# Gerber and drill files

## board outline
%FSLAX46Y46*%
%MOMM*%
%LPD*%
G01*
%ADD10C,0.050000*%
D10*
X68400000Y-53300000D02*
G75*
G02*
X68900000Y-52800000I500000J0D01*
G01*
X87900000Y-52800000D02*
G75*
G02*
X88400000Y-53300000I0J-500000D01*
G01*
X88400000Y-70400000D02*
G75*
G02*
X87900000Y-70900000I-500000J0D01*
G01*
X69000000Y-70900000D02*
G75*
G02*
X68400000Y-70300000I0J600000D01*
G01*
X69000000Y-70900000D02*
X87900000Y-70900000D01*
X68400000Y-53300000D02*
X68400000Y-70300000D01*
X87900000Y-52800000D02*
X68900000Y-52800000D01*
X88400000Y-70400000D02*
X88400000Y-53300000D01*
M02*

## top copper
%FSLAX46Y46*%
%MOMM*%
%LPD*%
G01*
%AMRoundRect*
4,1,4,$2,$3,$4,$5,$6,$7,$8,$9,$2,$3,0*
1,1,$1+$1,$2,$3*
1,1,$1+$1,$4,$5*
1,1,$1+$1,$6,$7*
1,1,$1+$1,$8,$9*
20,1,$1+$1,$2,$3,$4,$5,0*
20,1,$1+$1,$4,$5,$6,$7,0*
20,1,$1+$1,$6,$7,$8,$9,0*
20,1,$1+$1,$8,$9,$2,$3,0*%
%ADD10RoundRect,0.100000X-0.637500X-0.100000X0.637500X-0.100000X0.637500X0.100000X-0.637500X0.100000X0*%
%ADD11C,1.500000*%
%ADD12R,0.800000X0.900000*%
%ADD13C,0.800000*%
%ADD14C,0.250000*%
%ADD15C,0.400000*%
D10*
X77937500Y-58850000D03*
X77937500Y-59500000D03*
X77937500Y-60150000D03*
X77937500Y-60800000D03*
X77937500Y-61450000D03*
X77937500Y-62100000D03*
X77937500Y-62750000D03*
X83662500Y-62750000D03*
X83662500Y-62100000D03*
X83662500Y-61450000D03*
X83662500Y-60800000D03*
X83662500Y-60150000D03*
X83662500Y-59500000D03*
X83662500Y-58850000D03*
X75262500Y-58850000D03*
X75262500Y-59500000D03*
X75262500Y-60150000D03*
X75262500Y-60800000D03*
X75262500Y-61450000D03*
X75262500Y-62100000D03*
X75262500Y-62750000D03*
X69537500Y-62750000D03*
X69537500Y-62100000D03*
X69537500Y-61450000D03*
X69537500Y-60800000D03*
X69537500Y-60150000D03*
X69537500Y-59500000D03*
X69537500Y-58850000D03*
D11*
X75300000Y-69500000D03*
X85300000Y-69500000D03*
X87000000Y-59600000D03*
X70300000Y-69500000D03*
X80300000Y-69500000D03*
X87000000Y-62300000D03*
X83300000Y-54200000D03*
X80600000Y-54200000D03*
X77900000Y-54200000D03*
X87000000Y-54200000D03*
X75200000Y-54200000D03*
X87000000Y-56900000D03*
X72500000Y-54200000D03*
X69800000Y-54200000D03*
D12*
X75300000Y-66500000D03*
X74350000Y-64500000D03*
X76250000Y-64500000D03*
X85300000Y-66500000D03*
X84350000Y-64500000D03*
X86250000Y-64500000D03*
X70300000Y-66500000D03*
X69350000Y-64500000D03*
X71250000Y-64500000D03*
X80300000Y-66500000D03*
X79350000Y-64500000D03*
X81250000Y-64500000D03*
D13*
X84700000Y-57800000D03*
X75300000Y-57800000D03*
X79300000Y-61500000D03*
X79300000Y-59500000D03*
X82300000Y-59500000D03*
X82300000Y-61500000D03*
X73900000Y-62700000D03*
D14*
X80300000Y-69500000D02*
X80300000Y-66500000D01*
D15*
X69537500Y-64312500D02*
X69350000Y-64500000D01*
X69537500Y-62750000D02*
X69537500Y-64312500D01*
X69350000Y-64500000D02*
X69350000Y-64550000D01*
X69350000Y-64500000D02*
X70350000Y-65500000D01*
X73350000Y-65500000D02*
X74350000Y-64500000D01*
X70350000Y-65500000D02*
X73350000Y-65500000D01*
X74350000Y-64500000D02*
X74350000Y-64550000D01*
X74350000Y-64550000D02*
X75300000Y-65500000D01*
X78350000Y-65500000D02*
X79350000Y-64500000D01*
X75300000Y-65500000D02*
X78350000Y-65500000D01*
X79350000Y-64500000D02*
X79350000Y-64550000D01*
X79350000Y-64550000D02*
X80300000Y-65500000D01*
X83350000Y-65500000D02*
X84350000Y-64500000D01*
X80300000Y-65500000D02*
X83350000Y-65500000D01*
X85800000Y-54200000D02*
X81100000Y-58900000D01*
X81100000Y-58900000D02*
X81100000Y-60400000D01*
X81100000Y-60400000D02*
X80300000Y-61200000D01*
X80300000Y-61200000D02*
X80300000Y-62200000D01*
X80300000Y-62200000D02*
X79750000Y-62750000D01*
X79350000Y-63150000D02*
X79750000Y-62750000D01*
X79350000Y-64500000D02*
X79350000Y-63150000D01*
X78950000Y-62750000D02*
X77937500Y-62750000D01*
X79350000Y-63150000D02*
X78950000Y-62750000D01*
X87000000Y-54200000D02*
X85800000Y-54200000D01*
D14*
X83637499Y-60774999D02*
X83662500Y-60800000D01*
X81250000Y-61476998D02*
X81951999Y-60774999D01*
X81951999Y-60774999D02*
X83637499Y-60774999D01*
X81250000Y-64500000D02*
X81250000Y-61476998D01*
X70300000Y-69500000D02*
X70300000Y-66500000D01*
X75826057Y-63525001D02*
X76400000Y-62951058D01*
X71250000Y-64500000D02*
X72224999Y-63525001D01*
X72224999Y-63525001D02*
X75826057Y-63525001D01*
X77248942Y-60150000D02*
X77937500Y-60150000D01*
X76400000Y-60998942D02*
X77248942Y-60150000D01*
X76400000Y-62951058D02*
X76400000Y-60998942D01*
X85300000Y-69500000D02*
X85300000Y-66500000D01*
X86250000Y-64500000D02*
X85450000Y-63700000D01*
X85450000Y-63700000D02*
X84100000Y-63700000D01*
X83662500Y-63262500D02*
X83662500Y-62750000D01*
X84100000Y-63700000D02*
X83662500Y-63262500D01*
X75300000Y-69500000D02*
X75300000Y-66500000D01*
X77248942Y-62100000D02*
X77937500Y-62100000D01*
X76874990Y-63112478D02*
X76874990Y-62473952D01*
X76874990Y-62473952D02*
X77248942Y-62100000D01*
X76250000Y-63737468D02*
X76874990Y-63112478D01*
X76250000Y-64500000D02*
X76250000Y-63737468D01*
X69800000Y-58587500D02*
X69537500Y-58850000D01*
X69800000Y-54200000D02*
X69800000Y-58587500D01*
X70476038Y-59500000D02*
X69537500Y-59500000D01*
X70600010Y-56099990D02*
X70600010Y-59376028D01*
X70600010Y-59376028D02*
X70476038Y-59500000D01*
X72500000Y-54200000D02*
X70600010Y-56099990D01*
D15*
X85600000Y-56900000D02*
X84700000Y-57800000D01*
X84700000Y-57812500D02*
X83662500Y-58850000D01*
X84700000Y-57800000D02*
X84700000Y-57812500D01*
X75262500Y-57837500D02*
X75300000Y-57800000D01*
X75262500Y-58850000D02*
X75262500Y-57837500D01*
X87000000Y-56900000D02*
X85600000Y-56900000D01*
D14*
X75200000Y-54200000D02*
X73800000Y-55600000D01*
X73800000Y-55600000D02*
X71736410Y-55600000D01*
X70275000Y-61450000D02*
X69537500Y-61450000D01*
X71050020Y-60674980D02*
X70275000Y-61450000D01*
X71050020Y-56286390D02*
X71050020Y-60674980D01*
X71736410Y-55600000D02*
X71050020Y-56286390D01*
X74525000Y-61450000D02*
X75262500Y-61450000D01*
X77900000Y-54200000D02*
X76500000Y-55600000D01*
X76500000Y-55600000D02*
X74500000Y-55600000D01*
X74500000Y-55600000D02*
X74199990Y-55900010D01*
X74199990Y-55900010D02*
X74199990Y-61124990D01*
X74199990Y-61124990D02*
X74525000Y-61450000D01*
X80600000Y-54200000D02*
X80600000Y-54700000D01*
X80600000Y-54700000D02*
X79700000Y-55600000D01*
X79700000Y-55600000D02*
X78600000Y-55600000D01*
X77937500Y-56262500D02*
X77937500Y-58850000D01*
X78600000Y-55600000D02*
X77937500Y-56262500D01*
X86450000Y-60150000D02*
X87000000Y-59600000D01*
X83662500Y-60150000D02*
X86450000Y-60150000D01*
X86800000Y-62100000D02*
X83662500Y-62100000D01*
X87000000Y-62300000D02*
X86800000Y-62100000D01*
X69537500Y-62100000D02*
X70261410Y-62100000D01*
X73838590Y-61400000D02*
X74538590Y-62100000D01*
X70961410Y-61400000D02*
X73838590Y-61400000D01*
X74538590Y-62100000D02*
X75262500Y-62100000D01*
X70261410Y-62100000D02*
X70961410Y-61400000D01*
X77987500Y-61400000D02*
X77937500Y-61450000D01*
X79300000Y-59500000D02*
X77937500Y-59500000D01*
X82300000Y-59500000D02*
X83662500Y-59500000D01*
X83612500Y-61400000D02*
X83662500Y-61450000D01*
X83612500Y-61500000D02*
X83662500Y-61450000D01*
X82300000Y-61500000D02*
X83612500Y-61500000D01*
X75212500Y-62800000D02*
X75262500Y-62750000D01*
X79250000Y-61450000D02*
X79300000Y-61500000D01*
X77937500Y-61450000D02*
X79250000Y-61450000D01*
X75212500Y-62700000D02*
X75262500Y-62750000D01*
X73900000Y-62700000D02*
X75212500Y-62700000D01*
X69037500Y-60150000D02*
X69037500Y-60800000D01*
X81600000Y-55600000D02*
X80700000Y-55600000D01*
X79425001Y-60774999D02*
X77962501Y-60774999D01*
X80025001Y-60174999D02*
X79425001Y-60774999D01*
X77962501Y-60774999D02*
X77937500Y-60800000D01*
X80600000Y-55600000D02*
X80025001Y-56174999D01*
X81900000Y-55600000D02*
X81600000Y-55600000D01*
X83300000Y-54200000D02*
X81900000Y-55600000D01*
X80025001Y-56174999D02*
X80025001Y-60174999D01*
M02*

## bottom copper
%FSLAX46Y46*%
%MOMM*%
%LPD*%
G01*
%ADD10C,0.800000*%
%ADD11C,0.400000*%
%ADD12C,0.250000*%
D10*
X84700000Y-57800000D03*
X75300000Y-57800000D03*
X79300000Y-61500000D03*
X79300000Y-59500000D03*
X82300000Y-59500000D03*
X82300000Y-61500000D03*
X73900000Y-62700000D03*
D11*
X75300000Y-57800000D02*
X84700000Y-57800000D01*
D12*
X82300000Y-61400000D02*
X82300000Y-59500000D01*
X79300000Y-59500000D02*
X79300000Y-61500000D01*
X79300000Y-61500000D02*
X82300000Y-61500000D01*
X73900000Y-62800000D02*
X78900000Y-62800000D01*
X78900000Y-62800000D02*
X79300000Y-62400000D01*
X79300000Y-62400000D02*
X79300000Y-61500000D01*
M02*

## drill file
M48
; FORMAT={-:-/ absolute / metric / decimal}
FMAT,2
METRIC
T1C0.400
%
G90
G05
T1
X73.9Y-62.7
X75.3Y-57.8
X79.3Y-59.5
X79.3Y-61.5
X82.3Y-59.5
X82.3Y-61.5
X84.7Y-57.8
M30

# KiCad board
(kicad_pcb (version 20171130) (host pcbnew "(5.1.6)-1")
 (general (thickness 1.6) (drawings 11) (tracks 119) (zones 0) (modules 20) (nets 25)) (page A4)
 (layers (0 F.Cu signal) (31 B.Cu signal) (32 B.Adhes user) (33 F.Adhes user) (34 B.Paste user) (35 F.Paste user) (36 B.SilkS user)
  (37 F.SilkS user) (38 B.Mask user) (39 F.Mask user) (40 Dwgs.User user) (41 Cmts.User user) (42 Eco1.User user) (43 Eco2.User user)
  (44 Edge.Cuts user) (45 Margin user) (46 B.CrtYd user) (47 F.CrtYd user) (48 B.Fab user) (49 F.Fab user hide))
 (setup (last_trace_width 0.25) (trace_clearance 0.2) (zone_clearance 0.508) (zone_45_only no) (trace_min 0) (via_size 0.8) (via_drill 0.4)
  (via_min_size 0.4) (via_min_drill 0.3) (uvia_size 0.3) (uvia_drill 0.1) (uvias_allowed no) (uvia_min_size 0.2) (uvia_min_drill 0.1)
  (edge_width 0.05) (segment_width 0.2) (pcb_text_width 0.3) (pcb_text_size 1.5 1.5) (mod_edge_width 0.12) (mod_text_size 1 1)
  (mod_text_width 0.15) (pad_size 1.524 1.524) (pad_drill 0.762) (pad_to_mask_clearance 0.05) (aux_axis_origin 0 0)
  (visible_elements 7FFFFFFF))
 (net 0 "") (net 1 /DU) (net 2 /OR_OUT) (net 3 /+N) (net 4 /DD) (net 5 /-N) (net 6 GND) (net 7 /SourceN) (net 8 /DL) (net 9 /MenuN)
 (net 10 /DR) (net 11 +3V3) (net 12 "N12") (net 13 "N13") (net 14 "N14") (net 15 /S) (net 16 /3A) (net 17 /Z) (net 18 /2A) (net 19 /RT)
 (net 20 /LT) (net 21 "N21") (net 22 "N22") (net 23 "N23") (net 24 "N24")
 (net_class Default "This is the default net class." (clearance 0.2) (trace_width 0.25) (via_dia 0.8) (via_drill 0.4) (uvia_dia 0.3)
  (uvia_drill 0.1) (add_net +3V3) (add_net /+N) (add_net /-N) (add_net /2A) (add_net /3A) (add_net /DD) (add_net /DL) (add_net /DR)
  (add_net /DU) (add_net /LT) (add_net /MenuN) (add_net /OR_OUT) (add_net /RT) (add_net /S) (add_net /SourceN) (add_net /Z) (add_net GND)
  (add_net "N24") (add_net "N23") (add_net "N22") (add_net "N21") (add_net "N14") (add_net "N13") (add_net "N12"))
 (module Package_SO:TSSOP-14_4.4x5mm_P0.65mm (layer F.Cu) (at 80.8 60.8)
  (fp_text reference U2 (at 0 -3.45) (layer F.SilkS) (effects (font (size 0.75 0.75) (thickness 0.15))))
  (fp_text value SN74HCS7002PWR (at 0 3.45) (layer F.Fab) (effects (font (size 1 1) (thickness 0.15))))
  (pad 1 smd roundrect (at -2.8625 -1.95) (size 1.475 0.4) (layers F.Cu F.Paste F.Mask) (roundrect_rratio 0.25) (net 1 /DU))
  (pad 2 smd roundrect (at -2.8625 -1.3) (size 1.475 0.4) (layers F.Cu F.Paste F.Mask) (roundrect_rratio 0.25) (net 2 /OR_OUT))
  (pad 3 smd roundrect (at -2.8625 -0.65) (size 1.475 0.4) (layers F.Cu F.Paste F.Mask) (roundrect_rratio 0.25) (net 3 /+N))
  (pad 4 smd roundrect (at -2.8625 0) (size 1.475 0.4) (layers F.Cu F.Paste F.Mask) (roundrect_rratio 0.25) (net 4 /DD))
  (pad 5 smd roundrect (at -2.8625 0.65) (size 1.475 0.4) (layers F.Cu F.Paste F.Mask) (roundrect_rratio 0.25) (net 2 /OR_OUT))
  (pad 6 smd roundrect (at -2.8625 1.3) (size 1.475 0.4) (layers F.Cu F.Paste F.Mask) (roundrect_rratio 0.25) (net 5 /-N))
  (pad 7 smd roundrect (at -2.8625 1.95) (size 1.475 0.4) (layers F.Cu F.Paste F.Mask) (roundrect_rratio 0.25) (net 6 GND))
  (pad 8 smd roundrect (at 2.8625 1.95) (size 1.475 0.4) (layers F.Cu F.Paste F.Mask) (roundrect_rratio 0.25) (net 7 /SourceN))
  (pad 9 smd roundrect (at 2.8625 1.3) (size 1.475 0.4) (layers F.Cu F.Paste F.Mask) (roundrect_rratio 0.25) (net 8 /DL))
  (pad 10 smd roundrect (at 2.8625 0.65) (size 1.475 0.4) (layers F.Cu F.Paste F.Mask) (roundrect_rratio 0.25) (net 2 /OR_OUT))
  (pad 11 smd roundrect (at 2.8625 0) (size 1.475 0.4) (layers F.Cu F.Paste F.Mask) (roundrect_rratio 0.25) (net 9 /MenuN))
  (pad 12 smd roundrect (at 2.8625 -0.65) (size 1.475 0.4) (layers F.Cu F.Paste F.Mask) (roundrect_rratio 0.25) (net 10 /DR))
  (pad 13 smd roundrect (at 2.8625 -1.3) (size 1.475 0.4) (layers F.Cu F.Paste F.Mask) (roundrect_rratio 0.25) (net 2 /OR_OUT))
  (pad 14 smd roundrect (at 2.8625 -1.95) (size 1.475 0.4) (layers F.Cu F.Paste F.Mask) (roundrect_rratio 0.25) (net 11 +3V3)))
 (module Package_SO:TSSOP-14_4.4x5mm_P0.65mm (layer F.Cu) (at 72.4 60.8)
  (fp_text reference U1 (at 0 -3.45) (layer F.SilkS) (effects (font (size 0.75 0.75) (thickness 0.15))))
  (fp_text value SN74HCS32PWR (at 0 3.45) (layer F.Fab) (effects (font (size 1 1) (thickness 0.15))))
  (pad 14 smd roundrect (at 2.8625 -1.95) (size 1.475 0.4) (layers F.Cu F.Paste F.Mask) (roundrect_rratio 0.25) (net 11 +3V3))
  (pad 13 smd roundrect (at 2.8625 -1.3) (size 1.475 0.4) (layers F.Cu F.Paste F.Mask) (roundrect_rratio 0.25) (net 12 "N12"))
  (pad 12 smd roundrect (at 2.8625 -0.65) (size 1.475 0.4) (layers F.Cu F.Paste F.Mask) (roundrect_rratio 0.25) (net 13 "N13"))
  (pad 11 smd roundrect (at 2.8625 0) (size 1.475 0.4) (layers F.Cu F.Paste F.Mask) (roundrect_rratio 0.25) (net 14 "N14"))
  (pad 10 smd roundrect (at 2.8625 0.65) (size 1.475 0.4) (layers F.Cu F.Paste F.Mask) (roundrect_rratio 0.25) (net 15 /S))
  (pad 9 smd roundrect (at 2.8625 1.3) (size 1.475 0.4) (layers F.Cu F.Paste F.Mask) (roundrect_rratio 0.25) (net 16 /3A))
  (pad 8 smd roundrect (at 2.8625 1.95) (size 1.475 0.4) (layers F.Cu F.Paste F.Mask) (roundrect_rratio 0.25) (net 2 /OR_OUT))
  (pad 7 smd roundrect (at -2.8625 1.95) (size 1.475 0.4) (layers F.Cu F.Paste F.Mask) (roundrect_rratio 0.25) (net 6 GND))
  (pad 6 smd roundrect (at -2.8625 1.3) (size 1.475 0.4) (layers F.Cu F.Paste F.Mask) (roundrect_rratio 0.25) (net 16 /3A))
  (pad 5 smd roundrect (at -2.8625 0.65) (size 1.475 0.4) (layers F.Cu F.Paste F.Mask) (roundrect_rratio 0.25) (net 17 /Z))
  (pad 4 smd roundrect (at -2.8625 0) (size 1.475 0.4) (layers F.Cu F.Paste F.Mask) (roundrect_rratio 0.25) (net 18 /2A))
  (pad 3 smd roundrect (at -2.8625 -0.65) (size 1.475 0.4) (layers F.Cu F.Paste F.Mask) (roundrect_rratio 0.25) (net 18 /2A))
  (pad 2 smd roundrect (at -2.8625 -1.3) (size 1.475 0.4) (layers F.Cu F.Paste F.Mask) (roundrect_rratio 0.25) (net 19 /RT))
  (pad 1 smd roundrect (at -2.8625 -1.95) (size 1.475 0.4) (layers F.Cu F.Paste F.Mask) (roundrect_rratio 0.25) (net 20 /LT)))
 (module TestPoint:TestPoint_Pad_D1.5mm (layer F.Cu) (at 75.3 69.5)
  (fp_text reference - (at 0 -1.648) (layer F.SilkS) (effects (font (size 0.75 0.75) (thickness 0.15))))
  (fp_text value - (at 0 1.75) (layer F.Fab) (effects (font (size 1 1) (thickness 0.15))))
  (pad 1 smd circle (at 0 0) (size 1.5 1.5) (layers F.Cu F.Mask) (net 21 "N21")))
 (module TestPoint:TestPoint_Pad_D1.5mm (layer F.Cu) (at 85.3 69.5)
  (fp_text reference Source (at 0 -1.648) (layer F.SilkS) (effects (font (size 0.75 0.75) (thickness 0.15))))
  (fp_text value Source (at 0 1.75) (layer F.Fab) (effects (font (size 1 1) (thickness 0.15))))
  (pad 1 smd circle (at 0 0) (size 1.5 1.5) (layers F.Cu F.Mask) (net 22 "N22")))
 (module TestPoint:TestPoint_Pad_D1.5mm (layer F.Cu) (at 87 59.6 90)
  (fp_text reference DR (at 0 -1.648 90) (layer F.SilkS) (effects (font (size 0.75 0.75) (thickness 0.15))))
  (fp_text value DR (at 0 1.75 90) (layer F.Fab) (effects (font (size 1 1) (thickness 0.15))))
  (pad 1 smd circle (at 0 0 90) (size 1.5 1.5) (layers F.Cu F.Mask) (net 10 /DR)))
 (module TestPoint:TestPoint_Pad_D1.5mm (layer F.Cu) (at 70.3 69.5)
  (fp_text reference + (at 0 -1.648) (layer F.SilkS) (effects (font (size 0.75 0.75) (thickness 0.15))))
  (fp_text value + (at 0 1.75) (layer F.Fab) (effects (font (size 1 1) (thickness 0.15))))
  (pad 1 smd circle (at 0 0) (size 1.5 1.5) (layers F.Cu F.Mask) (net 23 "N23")))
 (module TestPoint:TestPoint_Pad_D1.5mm (layer F.Cu) (at 80.3 69.5)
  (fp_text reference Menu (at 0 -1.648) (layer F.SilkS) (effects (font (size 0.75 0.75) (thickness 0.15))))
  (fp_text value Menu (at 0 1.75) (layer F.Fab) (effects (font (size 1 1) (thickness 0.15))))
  (pad 1 smd circle (at 0 0) (size 1.5 1.5) (layers F.Cu F.Mask) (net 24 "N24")))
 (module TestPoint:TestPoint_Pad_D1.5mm (layer F.Cu) (at 87 62.3 90)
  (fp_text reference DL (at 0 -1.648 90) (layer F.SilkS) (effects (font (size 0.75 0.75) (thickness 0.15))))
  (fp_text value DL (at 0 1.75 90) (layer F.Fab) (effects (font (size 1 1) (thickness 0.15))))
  (pad 1 smd circle (at 0 0 90) (size 1.5 1.5) (layers F.Cu F.Mask) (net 8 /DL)))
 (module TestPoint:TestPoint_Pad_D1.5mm (layer F.Cu) (at 83.3 54.2 180)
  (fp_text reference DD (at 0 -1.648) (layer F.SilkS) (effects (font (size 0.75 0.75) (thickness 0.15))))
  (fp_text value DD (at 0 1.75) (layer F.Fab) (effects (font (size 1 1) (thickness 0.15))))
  (pad 1 smd circle (at 0 0 180) (size 1.5 1.5) (layers F.Cu F.Mask) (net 4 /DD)))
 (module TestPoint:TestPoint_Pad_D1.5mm (layer F.Cu) (at 80.6 54.2 180)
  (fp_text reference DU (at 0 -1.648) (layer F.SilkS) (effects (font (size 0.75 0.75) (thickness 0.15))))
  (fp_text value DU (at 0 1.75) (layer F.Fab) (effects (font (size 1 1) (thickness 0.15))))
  (pad 1 smd circle (at 0 0 180) (size 1.5 1.5) (layers F.Cu F.Mask) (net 1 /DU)))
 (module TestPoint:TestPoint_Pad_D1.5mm (layer F.Cu) (at 77.9 54.2 180)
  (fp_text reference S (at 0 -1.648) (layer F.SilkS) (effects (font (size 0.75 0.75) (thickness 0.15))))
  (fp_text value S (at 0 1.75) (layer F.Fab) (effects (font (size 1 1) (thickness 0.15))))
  (pad 1 smd circle (at 0 0 180) (size 1.5 1.5) (layers F.Cu F.Mask) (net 15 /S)))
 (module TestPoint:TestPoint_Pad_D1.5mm (layer F.Cu) (at 87 54.2 90)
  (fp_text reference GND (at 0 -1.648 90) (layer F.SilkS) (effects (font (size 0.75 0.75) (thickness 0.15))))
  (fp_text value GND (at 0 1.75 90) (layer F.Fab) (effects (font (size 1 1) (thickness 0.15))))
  (pad 1 smd circle (at 0 0 90) (size 1.5 1.5) (layers F.Cu F.Mask) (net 6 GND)))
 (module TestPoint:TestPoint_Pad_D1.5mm (layer F.Cu) (at 75.2 54.2 180)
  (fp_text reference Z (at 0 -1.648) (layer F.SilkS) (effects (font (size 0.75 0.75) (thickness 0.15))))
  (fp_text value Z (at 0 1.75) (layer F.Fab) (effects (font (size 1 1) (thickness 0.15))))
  (pad 1 smd circle (at 0 0 180) (size 1.5 1.5) (layers F.Cu F.Mask) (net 17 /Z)))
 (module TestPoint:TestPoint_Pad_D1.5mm (layer F.Cu) (at 87 56.9 90)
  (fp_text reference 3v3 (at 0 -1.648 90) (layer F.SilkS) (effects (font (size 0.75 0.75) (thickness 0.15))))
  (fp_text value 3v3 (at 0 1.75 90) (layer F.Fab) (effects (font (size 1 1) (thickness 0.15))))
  (pad 1 smd circle (at 0 0 90) (size 1.5 1.5) (layers F.Cu F.Mask) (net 11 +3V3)))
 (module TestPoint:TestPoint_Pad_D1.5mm (layer F.Cu) (at 72.5 54.2 180)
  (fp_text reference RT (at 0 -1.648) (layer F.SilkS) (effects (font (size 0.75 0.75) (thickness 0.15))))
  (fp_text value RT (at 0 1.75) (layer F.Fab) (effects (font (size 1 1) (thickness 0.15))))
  (pad 1 smd circle (at 0 0 180) (size 1.5 1.5) (layers F.Cu F.Mask) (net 19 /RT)))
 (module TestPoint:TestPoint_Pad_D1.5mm (layer F.Cu) (at 69.8 54.2 180)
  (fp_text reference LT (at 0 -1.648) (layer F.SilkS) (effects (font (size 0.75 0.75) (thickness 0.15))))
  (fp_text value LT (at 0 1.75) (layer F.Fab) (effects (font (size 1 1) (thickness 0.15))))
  (pad 1 smd circle (at 0 0 180) (size 1.5 1.5) (layers F.Cu F.Mask) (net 20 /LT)))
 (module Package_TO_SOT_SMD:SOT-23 (layer F.Cu) (at 75.3 65.5 270)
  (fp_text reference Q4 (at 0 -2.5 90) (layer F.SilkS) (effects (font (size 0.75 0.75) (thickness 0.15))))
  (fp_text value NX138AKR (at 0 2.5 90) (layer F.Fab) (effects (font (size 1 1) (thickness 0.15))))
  (pad 3 smd rect (at 1 0 270) (size 0.9 0.8) (layers F.Cu F.Paste F.Mask) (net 21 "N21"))
  (pad 2 smd rect (at -1 0.95 270) (size 0.9 0.8) (layers F.Cu F.Paste F.Mask) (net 6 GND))
  (pad 1 smd rect (at -1 -0.95 270) (size 0.9 0.8) (layers F.Cu F.Paste F.Mask) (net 5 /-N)))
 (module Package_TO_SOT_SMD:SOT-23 (layer F.Cu) (at 85.3 65.5 270)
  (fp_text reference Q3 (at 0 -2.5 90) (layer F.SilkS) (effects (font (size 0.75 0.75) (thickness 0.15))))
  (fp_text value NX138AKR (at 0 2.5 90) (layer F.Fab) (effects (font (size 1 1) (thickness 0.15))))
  (pad 3 smd rect (at 1 0 270) (size 0.9 0.8) (layers F.Cu F.Paste F.Mask) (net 22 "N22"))
  (pad 2 smd rect (at -1 0.95 270) (size 0.9 0.8) (layers F.Cu F.Paste F.Mask) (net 6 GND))
  (pad 1 smd rect (at -1 -0.95 270) (size 0.9 0.8) (layers F.Cu F.Paste F.Mask) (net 7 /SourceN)))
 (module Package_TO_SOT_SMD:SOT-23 (layer F.Cu) (at 70.3 65.5 270)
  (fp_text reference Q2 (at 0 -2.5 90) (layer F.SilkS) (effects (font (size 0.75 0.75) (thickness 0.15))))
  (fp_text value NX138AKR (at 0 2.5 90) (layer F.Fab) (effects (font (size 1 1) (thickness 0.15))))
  (pad 3 smd rect (at 1 0 270) (size 0.9 0.8) (layers F.Cu F.Paste F.Mask) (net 23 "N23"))
  (pad 2 smd rect (at -1 0.95 270) (size 0.9 0.8) (layers F.Cu F.Paste F.Mask) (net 6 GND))
  (pad 1 smd rect (at -1 -0.95 270) (size 0.9 0.8) (layers F.Cu F.Paste F.Mask) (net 3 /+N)))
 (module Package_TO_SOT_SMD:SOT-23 (layer F.Cu) (at 80.3 65.5 270)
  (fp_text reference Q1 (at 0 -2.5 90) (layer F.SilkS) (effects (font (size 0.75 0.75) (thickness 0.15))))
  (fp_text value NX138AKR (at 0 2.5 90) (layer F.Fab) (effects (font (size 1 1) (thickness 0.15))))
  (pad 3 smd rect (at 1 0 270) (size 0.9 0.8) (layers F.Cu F.Paste F.Mask) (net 24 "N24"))
  (pad 2 smd rect (at -1 0.95 270) (size 0.9 0.8) (layers F.Cu F.Paste F.Mask) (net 6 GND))
  (pad 1 smd rect (at -1 -0.95 270) (size 0.9 0.8) (layers F.Cu F.Paste F.Mask) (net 9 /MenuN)))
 (gr_arc (start 68.9 53.3) (end 68.9 52.8) (angle -90) (layer Edge.Cuts) (width 0.05))
 (gr_arc (start 87.9 53.3) (end 88.4 53.3) (angle -90) (layer Edge.Cuts) (width 0.05))
 (gr_arc (start 87.9 70.4) (end 87.9 70.9) (angle -90) (layer Edge.Cuts) (width 0.05))
 (gr_arc (start 69 70.3) (end 68.4 70.3) (angle -90) (layer Edge.Cuts) (width 0.05))
 (gr_line (start 69 70.9) (end 87.9 70.9) (layer Edge.Cuts) (width 0.05))
 (gr_line (start 68.4 53.3) (end 68.4 70.3) (layer Edge.Cuts) (width 0.05))
 (gr_line (start 87.9 52.8) (end 68.9 52.8) (layer Edge.Cuts) (width 0.05))
 (gr_line (start 88.4 70.4) (end 88.4 53.3) (layer Edge.Cuts) (width 0.05))
 (segment (start 80.3 69.5) (end 80.3 66.5) (width 0.25) (layer F.Cu) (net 24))
 (segment (start 69.5375 64.3125) (end 69.35 64.5) (width 0.4) (layer F.Cu) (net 6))
 (segment (start 69.5375 62.75) (end 69.5375 64.3125) (width 0.4) (layer F.Cu) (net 6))
 (segment (start 69.35 64.5) (end 69.35 64.55) (width 0.4) (layer F.Cu) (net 6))
 (segment (start 69.35 64.5) (end 70.35 65.5) (width 0.4) (layer F.Cu) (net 6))
 (segment (start 73.35 65.5) (end 74.35 64.5) (width 0.4) (layer F.Cu) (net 6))
 (segment (start 70.35 65.5) (end 73.35 65.5) (width 0.4) (layer F.Cu) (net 6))
 (segment (start 74.35 64.5) (end 74.35 64.55) (width 0.4) (layer F.Cu) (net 6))
 (segment (start 74.35 64.55) (end 75.3 65.5) (width 0.4) (layer F.Cu) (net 6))
 (segment (start 78.35 65.5) (end 79.35 64.5) (width 0.4) (layer F.Cu) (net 6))
 (segment (start 75.3 65.5) (end 78.35 65.5) (width 0.4) (layer F.Cu) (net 6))
 (segment (start 79.35 64.5) (end 79.35 64.55) (width 0.4) (layer F.Cu) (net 6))
 (segment (start 79.35 64.55) (end 80.3 65.5) (width 0.4) (layer F.Cu) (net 6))
 (segment (start 83.35 65.5) (end 84.35 64.5) (width 0.4) (layer F.Cu) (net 6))
 (segment (start 80.3 65.5) (end 83.35 65.5) (width 0.4) (layer F.Cu) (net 6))
 (segment (start 85.8 54.2) (end 81.1 58.9) (width 0.4) (layer F.Cu) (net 6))
 (segment (start 81.1 58.9) (end 81.1 60.4) (width 0.4) (layer F.Cu) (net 6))
 (segment (start 81.1 60.4) (end 80.3 61.2) (width 0.4) (layer F.Cu) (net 6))
 (segment (start 80.3 61.2) (end 80.3 62.2) (width 0.4) (layer F.Cu) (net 6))
 (segment (start 80.3 62.2) (end 79.75 62.75) (width 0.4) (layer F.Cu) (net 6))
 (segment (start 79.35 63.15) (end 79.75 62.75) (width 0.4) (layer F.Cu) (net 6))
 (segment (start 79.35 64.5) (end 79.35 63.15) (width 0.4) (layer F.Cu) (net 6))
 (segment (start 78.95 62.75) (end 77.9375 62.75) (width 0.4) (layer F.Cu) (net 6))
 (segment (start 79.35 63.15) (end 78.95 62.75) (width 0.4) (layer F.Cu) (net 6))
 (segment (start 87 54.2) (end 85.8 54.2) (width 0.4) (layer F.Cu) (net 6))
 (segment (start 83.637499 60.774999) (end 83.6625 60.8) (width 0.25) (layer F.Cu) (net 9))
 (segment (start 81.25 61.476998) (end 81.951999 60.774999) (width 0.25) (layer F.Cu) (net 9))
 (segment (start 81.951999 60.774999) (end 83.637499 60.774999) (width 0.25) (layer F.Cu) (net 9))
 (segment (start 81.25 64.5) (end 81.25 61.476998) (width 0.25) (layer F.Cu) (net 9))
 (via (at 84.7 57.8) (size 0.8) (drill 0.4) (layers F.Cu B.Cu) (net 11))
 (via (at 75.3 57.8) (size 0.8) (drill 0.4) (layers F.Cu B.Cu) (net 11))
 (segment (start 70.3 69.5) (end 70.3 66.5) (width 0.25) (layer F.Cu) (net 23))
 (segment (start 75.826057 63.525001) (end 76.4 62.951058) (width 0.25) (layer F.Cu) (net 3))
 (segment (start 71.25 64.5) (end 72.224999 63.525001) (width 0.25) (layer F.Cu) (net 3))
 (segment (start 72.224999 63.525001) (end 75.826057 63.525001) (width 0.25) (layer F.Cu) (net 3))
 (segment (start 77.248942 60.15) (end 77.9375 60.15) (width 0.25) (layer F.Cu) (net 3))
 (segment (start 76.4 60.998942) (end 77.248942 60.15) (width 0.25) (layer F.Cu) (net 3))
 (segment (start 76.4 62.951058) (end 76.4 60.998942) (width 0.25) (layer F.Cu) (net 3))
 (segment (start 85.3 69.5) (end 85.3 66.5) (width 0.25) (layer F.Cu) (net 22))
 (segment (start 86.25 64.5) (end 85.45 63.7) (width 0.25) (layer F.Cu) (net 7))
 (segment (start 85.45 63.7) (end 84.1 63.7) (width 0.25) (layer F.Cu) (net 7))
 (segment (start 83.6625 63.2625) (end 83.6625 62.75) (width 0.25) (layer F.Cu) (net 7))
 (segment (start 84.1 63.7) (end 83.6625 63.2625) (width 0.25) (layer F.Cu) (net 7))
 (segment (start 75.3 69.5) (end 75.3 66.5) (width 0.25) (layer F.Cu) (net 21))
 (segment (start 77.248942 62.1) (end 77.9375 62.1) (width 0.25) (layer F.Cu) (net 5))
 (segment (start 76.87499 63.112478) (end 76.87499 62.473952) (width 0.25) (layer F.Cu) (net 5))
 (segment (start 76.87499 62.473952) (end 77.248942 62.1) (width 0.25) (layer F.Cu) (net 5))
 (segment (start 76.25 63.737468) (end 76.87499 63.112478) (width 0.25) (layer F.Cu) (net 5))
 (segment (start 76.25 64.5) (end 76.25 63.737468) (width 0.25) (layer F.Cu) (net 5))
 (segment (start 69.8 58.5875) (end 69.5375 58.85) (width 0.25) (layer F.Cu) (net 20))
 (segment (start 69.8 54.2) (end 69.8 58.5875) (width 0.25) (layer F.Cu) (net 20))
 (segment (start 70.476038 59.5) (end 69.5375 59.5) (width 0.25) (layer F.Cu) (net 19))
 (segment (start 70.60001 56.09999) (end 70.60001 59.376028) (width 0.25) (layer F.Cu) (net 19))
 (segment (start 70.60001 59.376028) (end 70.476038 59.5) (width 0.25) (layer F.Cu) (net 19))
 (segment (start 72.5 54.2) (end 70.60001 56.09999) (width 0.25) (layer F.Cu) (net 19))
 (segment (start 85.6 56.9) (end 84.7 57.8) (width 0.4) (layer F.Cu) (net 11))
 (segment (start 84.7 57.8125) (end 83.6625 58.85) (width 0.4) (layer F.Cu) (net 11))
 (segment (start 84.7 57.8) (end 84.7 57.8125) (width 0.4) (layer F.Cu) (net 11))
 (segment (start 75.2625 57.8375) (end 75.3 57.8) (width 0.4) (layer F.Cu) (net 11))
 (segment (start 75.2625 58.85) (end 75.2625 57.8375) (width 0.4) (layer F.Cu) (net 11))
 (segment (start 75.3 57.8) (end 84.7 57.8) (width 0.4) (layer B.Cu) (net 11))
 (segment (start 87 56.9) (end 85.6 56.9) (width 0.4) (layer F.Cu) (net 11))
 (segment (start 75.2 54.2) (end 73.8 55.6) (width 0.25) (layer F.Cu) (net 17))
 (segment (start 73.8 55.6) (end 71.73641 55.6) (width 0.25) (layer F.Cu) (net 17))
 (segment (start 70.275 61.45) (end 69.5375 61.45) (width 0.25) (layer F.Cu) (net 17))
 (segment (start 71.05002 60.67498) (end 70.275 61.45) (width 0.25) (layer F.Cu) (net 17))
 (segment (start 71.05002 56.28639) (end 71.05002 60.67498) (width 0.25) (layer F.Cu) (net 17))
 (segment (start 71.73641 55.6) (end 71.05002 56.28639) (width 0.25) (layer F.Cu) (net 17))
 (segment (start 74.525 61.45) (end 75.2625 61.45) (width 0.25) (layer F.Cu) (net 15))
 (segment (start 77.9 54.2) (end 76.5 55.6) (width 0.25) (layer F.Cu) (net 15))
 (segment (start 76.5 55.6) (end 74.5 55.6) (width 0.25) (layer F.Cu) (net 15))
 (segment (start 74.5 55.6) (end 74.19999 55.90001) (width 0.25) (layer F.Cu) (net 15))
 (segment (start 74.19999 55.90001) (end 74.19999 61.12499) (width 0.25) (layer F.Cu) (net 15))
 (segment (start 74.19999 61.12499) (end 74.525 61.45) (width 0.25) (layer F.Cu) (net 15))
 (segment (start 80.6 54.2) (end 80.6 54.7) (width 0.25) (layer F.Cu) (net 1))
 (segment (start 80.6 54.7) (end 79.7 55.6) (width 0.25) (layer F.Cu) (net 1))
 (segment (start 79.7 55.6) (end 78.6 55.6) (width 0.25) (layer F.Cu) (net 1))
 (segment (start 77.9375 56.2625) (end 77.9375 58.85) (width 0.25) (layer F.Cu) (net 1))
 (segment (start 78.6 55.6) (end 77.9375 56.2625) (width 0.25) (layer F.Cu) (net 1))
 (segment (start 86.45 60.15) (end 87 59.6) (width 0.25) (layer F.Cu) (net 10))
 (segment (start 83.6625 60.15) (end 86.45 60.15) (width 0.25) (layer F.Cu) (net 10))
 (segment (start 86.8 62.1) (end 83.6625 62.1) (width 0.25) (layer F.Cu) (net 8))
 (segment (start 87 62.3) (end 86.8 62.1) (width 0.25) (layer F.Cu) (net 8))
 (segment (start 69.5375 62.1) (end 70.26141 62.1) (width 0.25) (layer F.Cu) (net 16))
 (segment (start 73.83859 61.4) (end 74.53859 62.1) (width 0.25) (layer F.Cu) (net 16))
 (segment (start 70.96141 61.4) (end 73.83859 61.4) (width 0.25) (layer F.Cu) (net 16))
 (segment (start 74.53859 62.1) (end 75.2625 62.1) (width 0.25) (layer F.Cu) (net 16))
 (segment (start 70.26141 62.1) (end 70.96141 61.4) (width 0.25) (layer F.Cu) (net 16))
 (via (at 79.3 61.5) (size 0.8) (drill 0.4) (layers F.Cu B.Cu) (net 2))
 (via (at 79.3 59.5) (size 0.8) (drill 0.4) (layers F.Cu B.Cu) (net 2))
 (via (at 82.3 59.5) (size 0.8) (drill 0.4) (layers F.Cu B.Cu) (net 2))
 (via (at 82.3 61.5) (size 0.8) (drill 0.4) (layers F.Cu B.Cu) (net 2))
 (via (at 73.9 62.7) (size 0.8) (drill 0.4) (layers F.Cu B.Cu) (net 2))
 (segment (start 77.9875 61.4) (end 77.9375 61.45) (width 0.25) (layer F.Cu) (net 2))
 (segment (start 79.3 59.5) (end 77.9375 59.5) (width 0.25) (layer F.Cu) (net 2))
 (segment (start 82.3 59.5) (end 83.6625 59.5) (width 0.25) (layer F.Cu) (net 2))
 (segment (start 83.6125 61.4) (end 83.6625 61.45) (width 0.25) (layer F.Cu) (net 2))
 (segment (start 82.3 61.4) (end 82.3 59.5) (width 0.25) (layer B.Cu) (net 2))
 (segment (start 83.6125 61.5) (end 83.6625 61.45) (width 0.25) (layer F.Cu) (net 2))
 (segment (start 82.3 61.5) (end 83.6125 61.5) (width 0.25) (layer F.Cu) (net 2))
 (segment (start 75.2125 62.8) (end 75.2625 62.75) (width 0.25) (layer F.Cu) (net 2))
 (segment (start 79.25 61.45) (end 79.3 61.5) (width 0.25) (layer F.Cu) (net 2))
 (segment (start 77.9375 61.45) (end 79.25 61.45) (width 0.25) (layer F.Cu) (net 2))
 (segment (start 79.3 59.5) (end 79.3 61.5) (width 0.25) (layer B.Cu) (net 2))
 (segment (start 79.3 61.5) (end 82.3 61.5) (width 0.25) (layer B.Cu) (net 2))
 (segment (start 73.9 62.8) (end 78.9 62.8) (width 0.25) (layer B.Cu) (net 2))
 (segment (start 78.9 62.8) (end 79.3 62.4) (width 0.25) (layer B.Cu) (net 2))
 (segment (start 79.3 62.4) (end 79.3 61.5) (width 0.25) (layer B.Cu) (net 2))
 (segment (start 75.2125 62.7) (end 75.2625 62.75) (width 0.25) (layer F.Cu) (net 2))
 (segment (start 73.9 62.7) (end 75.2125 62.7) (width 0.25) (layer F.Cu) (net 2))
 (segment (start 69.0375 60.15) (end 69.0375 60.8) (width 0.25) (layer F.Cu) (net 18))
 (segment (start 81.6 55.6) (end 80.7 55.6) (width 0.25) (layer F.Cu) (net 4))
 (segment (start 79.425001 60.774999) (end 77.962501 60.774999) (width 0.25) (layer F.Cu) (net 4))
 (segment (start 80.025001 60.174999) (end 79.425001 60.774999) (width 0.25) (layer F.Cu) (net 4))
 (segment (start 77.962501 60.774999) (end 77.9375 60.8) (width 0.25) (layer F.Cu) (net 4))
 (segment (start 80.6 55.6) (end 80.025001 56.174999) (width 0.25) (layer F.Cu) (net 4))
 (segment (start 81.9 55.6) (end 81.6 55.6) (width 0.25) (layer F.Cu) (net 4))
 (segment (start 83.3 54.2) (end 81.9 55.6) (width 0.25) (layer F.Cu) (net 4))
 (segment (start 80.025001 56.174999) (end 80.025001 60.174999) (width 0.25) (layer F.Cu) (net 4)))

